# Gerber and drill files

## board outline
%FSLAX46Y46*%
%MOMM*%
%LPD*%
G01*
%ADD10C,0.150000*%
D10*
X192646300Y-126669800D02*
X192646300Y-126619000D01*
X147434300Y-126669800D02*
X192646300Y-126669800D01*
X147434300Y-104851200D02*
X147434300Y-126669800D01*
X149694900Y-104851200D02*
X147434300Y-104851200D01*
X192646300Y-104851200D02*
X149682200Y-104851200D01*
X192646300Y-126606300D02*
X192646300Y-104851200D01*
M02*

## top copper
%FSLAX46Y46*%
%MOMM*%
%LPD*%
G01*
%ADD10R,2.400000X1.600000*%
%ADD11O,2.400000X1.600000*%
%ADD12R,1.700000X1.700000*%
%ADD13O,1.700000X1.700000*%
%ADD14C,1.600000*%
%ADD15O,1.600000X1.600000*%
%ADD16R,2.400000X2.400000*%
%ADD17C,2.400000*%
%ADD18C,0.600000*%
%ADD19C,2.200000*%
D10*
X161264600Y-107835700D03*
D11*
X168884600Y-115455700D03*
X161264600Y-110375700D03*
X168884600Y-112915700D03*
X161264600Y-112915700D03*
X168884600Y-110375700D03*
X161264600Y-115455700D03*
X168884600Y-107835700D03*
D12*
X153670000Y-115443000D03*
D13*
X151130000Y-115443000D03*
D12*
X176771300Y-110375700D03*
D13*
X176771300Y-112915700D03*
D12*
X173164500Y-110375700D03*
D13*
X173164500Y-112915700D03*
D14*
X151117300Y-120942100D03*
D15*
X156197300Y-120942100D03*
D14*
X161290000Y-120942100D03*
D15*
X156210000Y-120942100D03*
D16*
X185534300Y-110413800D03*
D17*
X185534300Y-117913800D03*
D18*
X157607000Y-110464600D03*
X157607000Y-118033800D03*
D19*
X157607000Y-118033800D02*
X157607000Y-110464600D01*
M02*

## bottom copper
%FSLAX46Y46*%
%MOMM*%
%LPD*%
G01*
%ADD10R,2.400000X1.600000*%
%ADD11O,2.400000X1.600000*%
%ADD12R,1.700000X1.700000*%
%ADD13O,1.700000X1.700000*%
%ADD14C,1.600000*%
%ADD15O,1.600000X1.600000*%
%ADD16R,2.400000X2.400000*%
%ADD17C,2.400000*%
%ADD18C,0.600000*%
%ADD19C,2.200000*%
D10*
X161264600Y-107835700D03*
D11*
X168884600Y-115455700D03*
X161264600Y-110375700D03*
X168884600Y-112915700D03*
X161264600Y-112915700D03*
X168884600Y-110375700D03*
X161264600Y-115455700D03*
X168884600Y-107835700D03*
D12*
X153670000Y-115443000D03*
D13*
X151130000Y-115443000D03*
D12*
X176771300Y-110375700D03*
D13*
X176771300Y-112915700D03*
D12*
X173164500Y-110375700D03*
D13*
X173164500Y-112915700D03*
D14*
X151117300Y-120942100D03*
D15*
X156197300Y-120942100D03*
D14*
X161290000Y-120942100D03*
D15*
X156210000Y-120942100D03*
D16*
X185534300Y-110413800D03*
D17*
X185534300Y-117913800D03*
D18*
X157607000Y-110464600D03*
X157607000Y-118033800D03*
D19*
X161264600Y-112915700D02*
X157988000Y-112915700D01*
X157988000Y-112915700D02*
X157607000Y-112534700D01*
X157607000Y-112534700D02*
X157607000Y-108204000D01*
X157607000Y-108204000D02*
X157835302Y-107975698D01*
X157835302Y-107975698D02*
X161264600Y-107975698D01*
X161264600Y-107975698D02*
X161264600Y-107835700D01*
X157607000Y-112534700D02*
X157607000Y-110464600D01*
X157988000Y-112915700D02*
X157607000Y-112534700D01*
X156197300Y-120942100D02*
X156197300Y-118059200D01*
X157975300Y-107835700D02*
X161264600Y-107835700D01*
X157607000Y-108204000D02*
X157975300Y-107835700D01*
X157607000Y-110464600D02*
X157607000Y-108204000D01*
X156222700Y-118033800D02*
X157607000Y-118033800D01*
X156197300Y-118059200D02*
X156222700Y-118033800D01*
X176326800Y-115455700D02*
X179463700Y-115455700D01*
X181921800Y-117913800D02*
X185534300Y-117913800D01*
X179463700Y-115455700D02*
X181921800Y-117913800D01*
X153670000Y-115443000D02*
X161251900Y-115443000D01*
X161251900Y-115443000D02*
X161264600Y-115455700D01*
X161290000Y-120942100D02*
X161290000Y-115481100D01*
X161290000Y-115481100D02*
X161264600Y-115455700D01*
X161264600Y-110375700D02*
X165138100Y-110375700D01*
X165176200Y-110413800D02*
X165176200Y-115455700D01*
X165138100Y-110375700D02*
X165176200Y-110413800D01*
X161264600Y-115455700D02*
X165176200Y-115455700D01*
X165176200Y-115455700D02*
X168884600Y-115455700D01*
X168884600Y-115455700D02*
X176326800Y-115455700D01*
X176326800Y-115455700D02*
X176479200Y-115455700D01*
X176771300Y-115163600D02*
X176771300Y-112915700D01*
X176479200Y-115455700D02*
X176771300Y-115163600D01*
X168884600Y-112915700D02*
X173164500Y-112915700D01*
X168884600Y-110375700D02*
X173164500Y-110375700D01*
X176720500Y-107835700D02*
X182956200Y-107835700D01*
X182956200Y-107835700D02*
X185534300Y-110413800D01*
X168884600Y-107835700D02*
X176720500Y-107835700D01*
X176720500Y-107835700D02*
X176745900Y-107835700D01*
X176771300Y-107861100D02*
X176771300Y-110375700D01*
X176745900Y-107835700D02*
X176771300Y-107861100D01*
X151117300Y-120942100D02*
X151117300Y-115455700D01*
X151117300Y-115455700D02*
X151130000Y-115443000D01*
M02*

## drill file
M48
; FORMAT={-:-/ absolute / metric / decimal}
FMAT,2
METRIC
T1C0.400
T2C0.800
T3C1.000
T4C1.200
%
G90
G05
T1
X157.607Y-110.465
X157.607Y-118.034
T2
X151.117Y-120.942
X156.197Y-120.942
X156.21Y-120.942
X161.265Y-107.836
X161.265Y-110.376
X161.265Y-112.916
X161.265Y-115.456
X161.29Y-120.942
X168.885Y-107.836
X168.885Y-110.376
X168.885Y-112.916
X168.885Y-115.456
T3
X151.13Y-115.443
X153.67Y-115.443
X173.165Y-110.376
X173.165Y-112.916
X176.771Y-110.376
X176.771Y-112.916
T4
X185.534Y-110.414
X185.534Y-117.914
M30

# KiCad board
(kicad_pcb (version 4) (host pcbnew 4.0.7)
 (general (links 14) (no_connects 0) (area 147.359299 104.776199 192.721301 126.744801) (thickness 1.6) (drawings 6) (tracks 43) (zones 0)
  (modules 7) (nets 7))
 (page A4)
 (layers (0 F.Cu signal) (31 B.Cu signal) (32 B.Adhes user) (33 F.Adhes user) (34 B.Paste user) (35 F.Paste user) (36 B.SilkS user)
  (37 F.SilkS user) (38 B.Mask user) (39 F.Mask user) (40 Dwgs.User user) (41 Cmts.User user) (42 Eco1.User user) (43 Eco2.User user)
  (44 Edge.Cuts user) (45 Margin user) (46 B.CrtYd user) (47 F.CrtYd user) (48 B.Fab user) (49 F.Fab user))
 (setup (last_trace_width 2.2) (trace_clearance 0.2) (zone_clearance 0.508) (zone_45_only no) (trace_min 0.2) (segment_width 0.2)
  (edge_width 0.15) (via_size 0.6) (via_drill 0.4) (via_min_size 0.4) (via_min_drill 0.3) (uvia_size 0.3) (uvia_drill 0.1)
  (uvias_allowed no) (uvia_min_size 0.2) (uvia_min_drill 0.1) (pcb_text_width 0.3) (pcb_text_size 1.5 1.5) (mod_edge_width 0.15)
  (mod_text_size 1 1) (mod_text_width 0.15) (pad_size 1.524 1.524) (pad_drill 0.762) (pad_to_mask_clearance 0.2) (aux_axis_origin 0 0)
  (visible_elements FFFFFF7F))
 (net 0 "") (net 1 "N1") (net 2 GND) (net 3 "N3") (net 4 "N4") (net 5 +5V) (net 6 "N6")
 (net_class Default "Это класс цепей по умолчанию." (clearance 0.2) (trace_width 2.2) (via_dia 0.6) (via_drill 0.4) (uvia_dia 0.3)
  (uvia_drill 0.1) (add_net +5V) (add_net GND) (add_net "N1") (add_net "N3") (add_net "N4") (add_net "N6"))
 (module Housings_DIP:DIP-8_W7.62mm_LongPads (layer F.Cu) (at 161.2646 107.8357)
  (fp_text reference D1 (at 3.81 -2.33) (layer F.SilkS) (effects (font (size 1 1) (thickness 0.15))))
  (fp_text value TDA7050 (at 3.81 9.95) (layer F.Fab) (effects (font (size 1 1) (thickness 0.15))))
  (pad 1 thru_hole rect (at 0 0) (size 2.4 1.6) (drill 0.8) (layers *.Cu *.Mask) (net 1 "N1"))
  (pad 5 thru_hole oval (at 7.62 7.62) (size 2.4 1.6) (drill 0.8) (layers *.Cu *.Mask) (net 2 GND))
  (pad 2 thru_hole oval (at 0 2.54) (size 2.4 1.6) (drill 0.8) (layers *.Cu *.Mask) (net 2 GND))
  (pad 6 thru_hole oval (at 7.62 5.08) (size 2.4 1.6) (drill 0.8) (layers *.Cu *.Mask) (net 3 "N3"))
  (pad 3 thru_hole oval (at 0 5.08) (size 2.4 1.6) (drill 0.8) (layers *.Cu *.Mask) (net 1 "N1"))
  (pad 7 thru_hole oval (at 7.62 2.54) (size 2.4 1.6) (drill 0.8) (layers *.Cu *.Mask) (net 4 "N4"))
  (pad 4 thru_hole oval (at 0 7.62) (size 2.4 1.6) (drill 0.8) (layers *.Cu *.Mask) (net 2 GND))
  (pad 8 thru_hole oval (at 7.62 0) (size 2.4 1.6) (drill 0.8) (layers *.Cu *.Mask) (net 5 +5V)))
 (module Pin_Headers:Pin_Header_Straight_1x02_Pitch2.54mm (layer F.Cu) (at 153.67 115.443 270)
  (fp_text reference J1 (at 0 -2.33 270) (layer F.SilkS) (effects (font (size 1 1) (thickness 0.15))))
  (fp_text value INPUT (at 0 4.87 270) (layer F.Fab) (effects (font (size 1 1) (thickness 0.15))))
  (pad 1 thru_hole rect (at 0 0 270) (size 1.7 1.7) (drill 1) (layers *.Cu *.Mask) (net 2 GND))
  (pad 2 thru_hole oval (at 0 2.54 270) (size 1.7 1.7) (drill 1) (layers *.Cu *.Mask) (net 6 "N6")))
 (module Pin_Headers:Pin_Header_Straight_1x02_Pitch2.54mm (layer F.Cu) (at 176.7713 110.3757)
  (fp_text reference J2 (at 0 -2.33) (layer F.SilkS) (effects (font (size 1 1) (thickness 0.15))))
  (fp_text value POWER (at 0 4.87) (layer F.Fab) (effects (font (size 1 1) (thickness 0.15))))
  (pad 1 thru_hole rect (at 0 0) (size 1.7 1.7) (drill 1) (layers *.Cu *.Mask) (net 5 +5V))
  (pad 2 thru_hole oval (at 0 2.54) (size 1.7 1.7) (drill 1) (layers *.Cu *.Mask) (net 2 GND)))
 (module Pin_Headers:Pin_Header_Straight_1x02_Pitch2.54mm (layer F.Cu) (at 173.1645 110.3757)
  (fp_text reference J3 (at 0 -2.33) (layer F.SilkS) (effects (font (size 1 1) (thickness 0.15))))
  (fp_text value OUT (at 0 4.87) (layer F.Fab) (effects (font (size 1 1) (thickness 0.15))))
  (pad 1 thru_hole rect (at 0 0) (size 1.7 1.7) (drill 1) (layers *.Cu *.Mask) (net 4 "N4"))
  (pad 2 thru_hole oval (at 0 2.54) (size 1.7 1.7) (drill 1) (layers *.Cu *.Mask) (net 3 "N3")))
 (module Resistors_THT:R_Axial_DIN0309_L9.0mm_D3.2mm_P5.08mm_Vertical (layer F.Cu) (at 151.1173 120.9421)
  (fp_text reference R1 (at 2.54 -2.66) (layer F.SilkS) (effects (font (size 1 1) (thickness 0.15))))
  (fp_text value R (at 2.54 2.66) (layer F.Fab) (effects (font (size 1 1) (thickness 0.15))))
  (pad 1 thru_hole circle (at 0 0) (size 1.6 1.6) (drill 0.8) (layers *.Cu *.Mask) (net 6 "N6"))
  (pad 2 thru_hole oval (at 5.08 0) (size 1.6 1.6) (drill 0.8) (layers *.Cu *.Mask) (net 1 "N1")))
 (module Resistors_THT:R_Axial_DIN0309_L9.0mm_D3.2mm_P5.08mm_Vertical (layer F.Cu) (at 161.29 120.9421 180)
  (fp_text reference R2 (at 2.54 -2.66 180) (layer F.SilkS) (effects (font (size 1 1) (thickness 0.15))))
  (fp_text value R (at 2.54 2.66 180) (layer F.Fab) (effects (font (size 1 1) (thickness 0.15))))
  (pad 1 thru_hole circle (at 0 0 180) (size 1.6 1.6) (drill 0.8) (layers *.Cu *.Mask) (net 2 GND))
  (pad 2 thru_hole oval (at 5.08 0 180) (size 1.6 1.6) (drill 0.8) (layers *.Cu *.Mask) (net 1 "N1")))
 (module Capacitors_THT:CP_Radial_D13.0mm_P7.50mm (layer F.Cu) (at 185.5343 110.4138 270)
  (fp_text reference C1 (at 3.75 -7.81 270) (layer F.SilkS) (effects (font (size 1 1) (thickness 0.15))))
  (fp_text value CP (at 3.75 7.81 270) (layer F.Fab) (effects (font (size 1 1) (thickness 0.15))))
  (pad 1 thru_hole rect (at 0 0 270) (size 2.4 2.4) (drill 1.2) (layers *.Cu *.Mask) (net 5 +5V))
  (pad 2 thru_hole circle (at 7.5 0 270) (size 2.4 2.4) (drill 1.2) (layers *.Cu *.Mask) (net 2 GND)))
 (gr_line (start 192.6463 126.6698) (end 192.6463 126.619) (angle 90) (layer Edge.Cuts) (width 0.15))
 (gr_line (start 147.4343 126.6698) (end 192.6463 126.6698) (angle 90) (layer Edge.Cuts) (width 0.15))
 (gr_line (start 147.4343 104.8512) (end 147.4343 126.6698) (angle 90) (layer Edge.Cuts) (width 0.15))
 (gr_line (start 149.6949 104.8512) (end 147.4343 104.8512) (angle 90) (layer Edge.Cuts) (width 0.15))
 (gr_line (start 192.6463 104.8512) (end 149.6822 104.8512) (angle 90) (layer Edge.Cuts) (width 0.15))
 (gr_line (start 192.6463 126.6063) (end 192.6463 104.8512) (angle 90) (layer Edge.Cuts) (width 0.15))
 (segment (start 161.2646 112.9157) (end 157.988 112.9157) (width 2.2) (layer B.Cu) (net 1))
 (segment (start 157.988 112.9157) (end 157.607 112.5347) (width 2.2) (layer B.Cu) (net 1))
 (segment (start 157.607 112.5347) (end 157.607 108.204) (width 2.2) (layer B.Cu) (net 1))
 (segment (start 157.607 108.204) (end 157.835302 107.975698) (width 2.2) (layer B.Cu) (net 1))
 (segment (start 157.835302 107.975698) (end 161.2646 107.975698) (width 2.2) (layer B.Cu) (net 1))
 (segment (start 161.2646 107.975698) (end 161.2646 107.8357) (width 2.2) (layer B.Cu) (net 1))
 (segment (start 157.607 112.5347) (end 157.607 110.4646) (width 2.2) (layer B.Cu) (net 1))
 (segment (start 157.988 112.9157) (end 157.607 112.5347) (width 2.2) (layer B.Cu) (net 1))
 (segment (start 156.1973 120.9421) (end 156.1973 118.0592) (width 2.2) (layer B.Cu) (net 1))
 (segment (start 157.9753 107.8357) (end 161.2646 107.8357) (width 2.2) (layer B.Cu) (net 1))
 (segment (start 157.607 108.204) (end 157.9753 107.8357) (width 2.2) (layer B.Cu) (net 1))
 (segment (start 157.607 110.4646) (end 157.607 108.204) (width 2.2) (layer B.Cu) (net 1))
 (via (at 157.607 110.4646) (size 0.6) (drill 0.4) (layers F.Cu B.Cu) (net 1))
 (segment (start 157.607 118.0338) (end 157.607 110.4646) (width 2.2) (layer F.Cu) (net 1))
 (via (at 157.607 118.0338) (size 0.6) (drill 0.4) (layers F.Cu B.Cu) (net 1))
 (segment (start 156.2227 118.0338) (end 157.607 118.0338) (width 2.2) (layer B.Cu) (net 1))
 (segment (start 156.1973 118.0592) (end 156.2227 118.0338) (width 2.2) (layer B.Cu) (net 1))
 (segment (start 176.3268 115.4557) (end 179.4637 115.4557) (width 2.2) (layer B.Cu) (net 2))
 (segment (start 181.9218 117.9138) (end 185.5343 117.9138) (width 2.2) (layer B.Cu) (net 2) (status 800000))
 (segment (start 179.4637 115.4557) (end 181.9218 117.9138) (width 2.2) (layer B.Cu) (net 2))
 (segment (start 153.67 115.443) (end 161.2519 115.443) (width 2.2) (layer B.Cu) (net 2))
 (segment (start 161.2519 115.443) (end 161.2646 115.4557) (width 2.2) (layer B.Cu) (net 2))
 (segment (start 161.29 120.9421) (end 161.29 115.4811) (width 2.2) (layer B.Cu) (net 2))
 (segment (start 161.29 115.4811) (end 161.2646 115.4557) (width 2.2) (layer B.Cu) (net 2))
 (segment (start 161.2646 110.3757) (end 165.1381 110.3757) (width 2.2) (layer B.Cu) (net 2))
 (segment (start 165.1762 110.4138) (end 165.1762 115.4557) (width 2.2) (layer B.Cu) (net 2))
 (segment (start 165.1381 110.3757) (end 165.1762 110.4138) (width 2.2) (layer B.Cu) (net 2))
 (segment (start 161.2646 115.4557) (end 165.1762 115.4557) (width 2.2) (layer B.Cu) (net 2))
 (segment (start 165.1762 115.4557) (end 168.8846 115.4557) (width 2.2) (layer B.Cu) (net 2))
 (segment (start 168.8846 115.4557) (end 176.3268 115.4557) (width 2.2) (layer B.Cu) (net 2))
 (segment (start 176.3268 115.4557) (end 176.4792 115.4557) (width 2.2) (layer B.Cu) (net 2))
 (segment (start 176.7713 115.1636) (end 176.7713 112.9157) (width 2.2) (layer B.Cu) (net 2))
 (segment (start 176.4792 115.4557) (end 176.7713 115.1636) (width 2.2) (layer B.Cu) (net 2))
 (segment (start 168.8846 112.9157) (end 173.1645 112.9157) (width 2.2) (layer B.Cu) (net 3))
 (segment (start 168.8846 110.3757) (end 173.1645 110.3757) (width 2.2) (layer B.Cu) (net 4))
 (segment (start 176.7205 107.8357) (end 182.9562 107.8357) (width 2.2) (layer B.Cu) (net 5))
 (segment (start 182.9562 107.8357) (end 185.5343 110.4138) (width 2.2) (layer B.Cu) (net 5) (status 800000))
 (segment (start 168.8846 107.8357) (end 176.7205 107.8357) (width 2.2) (layer B.Cu) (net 5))
 (segment (start 176.7205 107.8357) (end 176.7459 107.8357) (width 2.2) (layer B.Cu) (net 5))
 (segment (start 176.7713 107.8611) (end 176.7713 110.3757) (width 2.2) (layer B.Cu) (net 5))
 (segment (start 176.7459 107.8357) (end 176.7713 107.8611) (width 2.2) (layer B.Cu) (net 5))
 (segment (start 151.1173 120.9421) (end 151.1173 115.4557) (width 2.2) (layer B.Cu) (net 6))
 (segment (start 151.1173 115.4557) (end 151.13 115.443) (width 2.2) (layer B.Cu) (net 6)))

